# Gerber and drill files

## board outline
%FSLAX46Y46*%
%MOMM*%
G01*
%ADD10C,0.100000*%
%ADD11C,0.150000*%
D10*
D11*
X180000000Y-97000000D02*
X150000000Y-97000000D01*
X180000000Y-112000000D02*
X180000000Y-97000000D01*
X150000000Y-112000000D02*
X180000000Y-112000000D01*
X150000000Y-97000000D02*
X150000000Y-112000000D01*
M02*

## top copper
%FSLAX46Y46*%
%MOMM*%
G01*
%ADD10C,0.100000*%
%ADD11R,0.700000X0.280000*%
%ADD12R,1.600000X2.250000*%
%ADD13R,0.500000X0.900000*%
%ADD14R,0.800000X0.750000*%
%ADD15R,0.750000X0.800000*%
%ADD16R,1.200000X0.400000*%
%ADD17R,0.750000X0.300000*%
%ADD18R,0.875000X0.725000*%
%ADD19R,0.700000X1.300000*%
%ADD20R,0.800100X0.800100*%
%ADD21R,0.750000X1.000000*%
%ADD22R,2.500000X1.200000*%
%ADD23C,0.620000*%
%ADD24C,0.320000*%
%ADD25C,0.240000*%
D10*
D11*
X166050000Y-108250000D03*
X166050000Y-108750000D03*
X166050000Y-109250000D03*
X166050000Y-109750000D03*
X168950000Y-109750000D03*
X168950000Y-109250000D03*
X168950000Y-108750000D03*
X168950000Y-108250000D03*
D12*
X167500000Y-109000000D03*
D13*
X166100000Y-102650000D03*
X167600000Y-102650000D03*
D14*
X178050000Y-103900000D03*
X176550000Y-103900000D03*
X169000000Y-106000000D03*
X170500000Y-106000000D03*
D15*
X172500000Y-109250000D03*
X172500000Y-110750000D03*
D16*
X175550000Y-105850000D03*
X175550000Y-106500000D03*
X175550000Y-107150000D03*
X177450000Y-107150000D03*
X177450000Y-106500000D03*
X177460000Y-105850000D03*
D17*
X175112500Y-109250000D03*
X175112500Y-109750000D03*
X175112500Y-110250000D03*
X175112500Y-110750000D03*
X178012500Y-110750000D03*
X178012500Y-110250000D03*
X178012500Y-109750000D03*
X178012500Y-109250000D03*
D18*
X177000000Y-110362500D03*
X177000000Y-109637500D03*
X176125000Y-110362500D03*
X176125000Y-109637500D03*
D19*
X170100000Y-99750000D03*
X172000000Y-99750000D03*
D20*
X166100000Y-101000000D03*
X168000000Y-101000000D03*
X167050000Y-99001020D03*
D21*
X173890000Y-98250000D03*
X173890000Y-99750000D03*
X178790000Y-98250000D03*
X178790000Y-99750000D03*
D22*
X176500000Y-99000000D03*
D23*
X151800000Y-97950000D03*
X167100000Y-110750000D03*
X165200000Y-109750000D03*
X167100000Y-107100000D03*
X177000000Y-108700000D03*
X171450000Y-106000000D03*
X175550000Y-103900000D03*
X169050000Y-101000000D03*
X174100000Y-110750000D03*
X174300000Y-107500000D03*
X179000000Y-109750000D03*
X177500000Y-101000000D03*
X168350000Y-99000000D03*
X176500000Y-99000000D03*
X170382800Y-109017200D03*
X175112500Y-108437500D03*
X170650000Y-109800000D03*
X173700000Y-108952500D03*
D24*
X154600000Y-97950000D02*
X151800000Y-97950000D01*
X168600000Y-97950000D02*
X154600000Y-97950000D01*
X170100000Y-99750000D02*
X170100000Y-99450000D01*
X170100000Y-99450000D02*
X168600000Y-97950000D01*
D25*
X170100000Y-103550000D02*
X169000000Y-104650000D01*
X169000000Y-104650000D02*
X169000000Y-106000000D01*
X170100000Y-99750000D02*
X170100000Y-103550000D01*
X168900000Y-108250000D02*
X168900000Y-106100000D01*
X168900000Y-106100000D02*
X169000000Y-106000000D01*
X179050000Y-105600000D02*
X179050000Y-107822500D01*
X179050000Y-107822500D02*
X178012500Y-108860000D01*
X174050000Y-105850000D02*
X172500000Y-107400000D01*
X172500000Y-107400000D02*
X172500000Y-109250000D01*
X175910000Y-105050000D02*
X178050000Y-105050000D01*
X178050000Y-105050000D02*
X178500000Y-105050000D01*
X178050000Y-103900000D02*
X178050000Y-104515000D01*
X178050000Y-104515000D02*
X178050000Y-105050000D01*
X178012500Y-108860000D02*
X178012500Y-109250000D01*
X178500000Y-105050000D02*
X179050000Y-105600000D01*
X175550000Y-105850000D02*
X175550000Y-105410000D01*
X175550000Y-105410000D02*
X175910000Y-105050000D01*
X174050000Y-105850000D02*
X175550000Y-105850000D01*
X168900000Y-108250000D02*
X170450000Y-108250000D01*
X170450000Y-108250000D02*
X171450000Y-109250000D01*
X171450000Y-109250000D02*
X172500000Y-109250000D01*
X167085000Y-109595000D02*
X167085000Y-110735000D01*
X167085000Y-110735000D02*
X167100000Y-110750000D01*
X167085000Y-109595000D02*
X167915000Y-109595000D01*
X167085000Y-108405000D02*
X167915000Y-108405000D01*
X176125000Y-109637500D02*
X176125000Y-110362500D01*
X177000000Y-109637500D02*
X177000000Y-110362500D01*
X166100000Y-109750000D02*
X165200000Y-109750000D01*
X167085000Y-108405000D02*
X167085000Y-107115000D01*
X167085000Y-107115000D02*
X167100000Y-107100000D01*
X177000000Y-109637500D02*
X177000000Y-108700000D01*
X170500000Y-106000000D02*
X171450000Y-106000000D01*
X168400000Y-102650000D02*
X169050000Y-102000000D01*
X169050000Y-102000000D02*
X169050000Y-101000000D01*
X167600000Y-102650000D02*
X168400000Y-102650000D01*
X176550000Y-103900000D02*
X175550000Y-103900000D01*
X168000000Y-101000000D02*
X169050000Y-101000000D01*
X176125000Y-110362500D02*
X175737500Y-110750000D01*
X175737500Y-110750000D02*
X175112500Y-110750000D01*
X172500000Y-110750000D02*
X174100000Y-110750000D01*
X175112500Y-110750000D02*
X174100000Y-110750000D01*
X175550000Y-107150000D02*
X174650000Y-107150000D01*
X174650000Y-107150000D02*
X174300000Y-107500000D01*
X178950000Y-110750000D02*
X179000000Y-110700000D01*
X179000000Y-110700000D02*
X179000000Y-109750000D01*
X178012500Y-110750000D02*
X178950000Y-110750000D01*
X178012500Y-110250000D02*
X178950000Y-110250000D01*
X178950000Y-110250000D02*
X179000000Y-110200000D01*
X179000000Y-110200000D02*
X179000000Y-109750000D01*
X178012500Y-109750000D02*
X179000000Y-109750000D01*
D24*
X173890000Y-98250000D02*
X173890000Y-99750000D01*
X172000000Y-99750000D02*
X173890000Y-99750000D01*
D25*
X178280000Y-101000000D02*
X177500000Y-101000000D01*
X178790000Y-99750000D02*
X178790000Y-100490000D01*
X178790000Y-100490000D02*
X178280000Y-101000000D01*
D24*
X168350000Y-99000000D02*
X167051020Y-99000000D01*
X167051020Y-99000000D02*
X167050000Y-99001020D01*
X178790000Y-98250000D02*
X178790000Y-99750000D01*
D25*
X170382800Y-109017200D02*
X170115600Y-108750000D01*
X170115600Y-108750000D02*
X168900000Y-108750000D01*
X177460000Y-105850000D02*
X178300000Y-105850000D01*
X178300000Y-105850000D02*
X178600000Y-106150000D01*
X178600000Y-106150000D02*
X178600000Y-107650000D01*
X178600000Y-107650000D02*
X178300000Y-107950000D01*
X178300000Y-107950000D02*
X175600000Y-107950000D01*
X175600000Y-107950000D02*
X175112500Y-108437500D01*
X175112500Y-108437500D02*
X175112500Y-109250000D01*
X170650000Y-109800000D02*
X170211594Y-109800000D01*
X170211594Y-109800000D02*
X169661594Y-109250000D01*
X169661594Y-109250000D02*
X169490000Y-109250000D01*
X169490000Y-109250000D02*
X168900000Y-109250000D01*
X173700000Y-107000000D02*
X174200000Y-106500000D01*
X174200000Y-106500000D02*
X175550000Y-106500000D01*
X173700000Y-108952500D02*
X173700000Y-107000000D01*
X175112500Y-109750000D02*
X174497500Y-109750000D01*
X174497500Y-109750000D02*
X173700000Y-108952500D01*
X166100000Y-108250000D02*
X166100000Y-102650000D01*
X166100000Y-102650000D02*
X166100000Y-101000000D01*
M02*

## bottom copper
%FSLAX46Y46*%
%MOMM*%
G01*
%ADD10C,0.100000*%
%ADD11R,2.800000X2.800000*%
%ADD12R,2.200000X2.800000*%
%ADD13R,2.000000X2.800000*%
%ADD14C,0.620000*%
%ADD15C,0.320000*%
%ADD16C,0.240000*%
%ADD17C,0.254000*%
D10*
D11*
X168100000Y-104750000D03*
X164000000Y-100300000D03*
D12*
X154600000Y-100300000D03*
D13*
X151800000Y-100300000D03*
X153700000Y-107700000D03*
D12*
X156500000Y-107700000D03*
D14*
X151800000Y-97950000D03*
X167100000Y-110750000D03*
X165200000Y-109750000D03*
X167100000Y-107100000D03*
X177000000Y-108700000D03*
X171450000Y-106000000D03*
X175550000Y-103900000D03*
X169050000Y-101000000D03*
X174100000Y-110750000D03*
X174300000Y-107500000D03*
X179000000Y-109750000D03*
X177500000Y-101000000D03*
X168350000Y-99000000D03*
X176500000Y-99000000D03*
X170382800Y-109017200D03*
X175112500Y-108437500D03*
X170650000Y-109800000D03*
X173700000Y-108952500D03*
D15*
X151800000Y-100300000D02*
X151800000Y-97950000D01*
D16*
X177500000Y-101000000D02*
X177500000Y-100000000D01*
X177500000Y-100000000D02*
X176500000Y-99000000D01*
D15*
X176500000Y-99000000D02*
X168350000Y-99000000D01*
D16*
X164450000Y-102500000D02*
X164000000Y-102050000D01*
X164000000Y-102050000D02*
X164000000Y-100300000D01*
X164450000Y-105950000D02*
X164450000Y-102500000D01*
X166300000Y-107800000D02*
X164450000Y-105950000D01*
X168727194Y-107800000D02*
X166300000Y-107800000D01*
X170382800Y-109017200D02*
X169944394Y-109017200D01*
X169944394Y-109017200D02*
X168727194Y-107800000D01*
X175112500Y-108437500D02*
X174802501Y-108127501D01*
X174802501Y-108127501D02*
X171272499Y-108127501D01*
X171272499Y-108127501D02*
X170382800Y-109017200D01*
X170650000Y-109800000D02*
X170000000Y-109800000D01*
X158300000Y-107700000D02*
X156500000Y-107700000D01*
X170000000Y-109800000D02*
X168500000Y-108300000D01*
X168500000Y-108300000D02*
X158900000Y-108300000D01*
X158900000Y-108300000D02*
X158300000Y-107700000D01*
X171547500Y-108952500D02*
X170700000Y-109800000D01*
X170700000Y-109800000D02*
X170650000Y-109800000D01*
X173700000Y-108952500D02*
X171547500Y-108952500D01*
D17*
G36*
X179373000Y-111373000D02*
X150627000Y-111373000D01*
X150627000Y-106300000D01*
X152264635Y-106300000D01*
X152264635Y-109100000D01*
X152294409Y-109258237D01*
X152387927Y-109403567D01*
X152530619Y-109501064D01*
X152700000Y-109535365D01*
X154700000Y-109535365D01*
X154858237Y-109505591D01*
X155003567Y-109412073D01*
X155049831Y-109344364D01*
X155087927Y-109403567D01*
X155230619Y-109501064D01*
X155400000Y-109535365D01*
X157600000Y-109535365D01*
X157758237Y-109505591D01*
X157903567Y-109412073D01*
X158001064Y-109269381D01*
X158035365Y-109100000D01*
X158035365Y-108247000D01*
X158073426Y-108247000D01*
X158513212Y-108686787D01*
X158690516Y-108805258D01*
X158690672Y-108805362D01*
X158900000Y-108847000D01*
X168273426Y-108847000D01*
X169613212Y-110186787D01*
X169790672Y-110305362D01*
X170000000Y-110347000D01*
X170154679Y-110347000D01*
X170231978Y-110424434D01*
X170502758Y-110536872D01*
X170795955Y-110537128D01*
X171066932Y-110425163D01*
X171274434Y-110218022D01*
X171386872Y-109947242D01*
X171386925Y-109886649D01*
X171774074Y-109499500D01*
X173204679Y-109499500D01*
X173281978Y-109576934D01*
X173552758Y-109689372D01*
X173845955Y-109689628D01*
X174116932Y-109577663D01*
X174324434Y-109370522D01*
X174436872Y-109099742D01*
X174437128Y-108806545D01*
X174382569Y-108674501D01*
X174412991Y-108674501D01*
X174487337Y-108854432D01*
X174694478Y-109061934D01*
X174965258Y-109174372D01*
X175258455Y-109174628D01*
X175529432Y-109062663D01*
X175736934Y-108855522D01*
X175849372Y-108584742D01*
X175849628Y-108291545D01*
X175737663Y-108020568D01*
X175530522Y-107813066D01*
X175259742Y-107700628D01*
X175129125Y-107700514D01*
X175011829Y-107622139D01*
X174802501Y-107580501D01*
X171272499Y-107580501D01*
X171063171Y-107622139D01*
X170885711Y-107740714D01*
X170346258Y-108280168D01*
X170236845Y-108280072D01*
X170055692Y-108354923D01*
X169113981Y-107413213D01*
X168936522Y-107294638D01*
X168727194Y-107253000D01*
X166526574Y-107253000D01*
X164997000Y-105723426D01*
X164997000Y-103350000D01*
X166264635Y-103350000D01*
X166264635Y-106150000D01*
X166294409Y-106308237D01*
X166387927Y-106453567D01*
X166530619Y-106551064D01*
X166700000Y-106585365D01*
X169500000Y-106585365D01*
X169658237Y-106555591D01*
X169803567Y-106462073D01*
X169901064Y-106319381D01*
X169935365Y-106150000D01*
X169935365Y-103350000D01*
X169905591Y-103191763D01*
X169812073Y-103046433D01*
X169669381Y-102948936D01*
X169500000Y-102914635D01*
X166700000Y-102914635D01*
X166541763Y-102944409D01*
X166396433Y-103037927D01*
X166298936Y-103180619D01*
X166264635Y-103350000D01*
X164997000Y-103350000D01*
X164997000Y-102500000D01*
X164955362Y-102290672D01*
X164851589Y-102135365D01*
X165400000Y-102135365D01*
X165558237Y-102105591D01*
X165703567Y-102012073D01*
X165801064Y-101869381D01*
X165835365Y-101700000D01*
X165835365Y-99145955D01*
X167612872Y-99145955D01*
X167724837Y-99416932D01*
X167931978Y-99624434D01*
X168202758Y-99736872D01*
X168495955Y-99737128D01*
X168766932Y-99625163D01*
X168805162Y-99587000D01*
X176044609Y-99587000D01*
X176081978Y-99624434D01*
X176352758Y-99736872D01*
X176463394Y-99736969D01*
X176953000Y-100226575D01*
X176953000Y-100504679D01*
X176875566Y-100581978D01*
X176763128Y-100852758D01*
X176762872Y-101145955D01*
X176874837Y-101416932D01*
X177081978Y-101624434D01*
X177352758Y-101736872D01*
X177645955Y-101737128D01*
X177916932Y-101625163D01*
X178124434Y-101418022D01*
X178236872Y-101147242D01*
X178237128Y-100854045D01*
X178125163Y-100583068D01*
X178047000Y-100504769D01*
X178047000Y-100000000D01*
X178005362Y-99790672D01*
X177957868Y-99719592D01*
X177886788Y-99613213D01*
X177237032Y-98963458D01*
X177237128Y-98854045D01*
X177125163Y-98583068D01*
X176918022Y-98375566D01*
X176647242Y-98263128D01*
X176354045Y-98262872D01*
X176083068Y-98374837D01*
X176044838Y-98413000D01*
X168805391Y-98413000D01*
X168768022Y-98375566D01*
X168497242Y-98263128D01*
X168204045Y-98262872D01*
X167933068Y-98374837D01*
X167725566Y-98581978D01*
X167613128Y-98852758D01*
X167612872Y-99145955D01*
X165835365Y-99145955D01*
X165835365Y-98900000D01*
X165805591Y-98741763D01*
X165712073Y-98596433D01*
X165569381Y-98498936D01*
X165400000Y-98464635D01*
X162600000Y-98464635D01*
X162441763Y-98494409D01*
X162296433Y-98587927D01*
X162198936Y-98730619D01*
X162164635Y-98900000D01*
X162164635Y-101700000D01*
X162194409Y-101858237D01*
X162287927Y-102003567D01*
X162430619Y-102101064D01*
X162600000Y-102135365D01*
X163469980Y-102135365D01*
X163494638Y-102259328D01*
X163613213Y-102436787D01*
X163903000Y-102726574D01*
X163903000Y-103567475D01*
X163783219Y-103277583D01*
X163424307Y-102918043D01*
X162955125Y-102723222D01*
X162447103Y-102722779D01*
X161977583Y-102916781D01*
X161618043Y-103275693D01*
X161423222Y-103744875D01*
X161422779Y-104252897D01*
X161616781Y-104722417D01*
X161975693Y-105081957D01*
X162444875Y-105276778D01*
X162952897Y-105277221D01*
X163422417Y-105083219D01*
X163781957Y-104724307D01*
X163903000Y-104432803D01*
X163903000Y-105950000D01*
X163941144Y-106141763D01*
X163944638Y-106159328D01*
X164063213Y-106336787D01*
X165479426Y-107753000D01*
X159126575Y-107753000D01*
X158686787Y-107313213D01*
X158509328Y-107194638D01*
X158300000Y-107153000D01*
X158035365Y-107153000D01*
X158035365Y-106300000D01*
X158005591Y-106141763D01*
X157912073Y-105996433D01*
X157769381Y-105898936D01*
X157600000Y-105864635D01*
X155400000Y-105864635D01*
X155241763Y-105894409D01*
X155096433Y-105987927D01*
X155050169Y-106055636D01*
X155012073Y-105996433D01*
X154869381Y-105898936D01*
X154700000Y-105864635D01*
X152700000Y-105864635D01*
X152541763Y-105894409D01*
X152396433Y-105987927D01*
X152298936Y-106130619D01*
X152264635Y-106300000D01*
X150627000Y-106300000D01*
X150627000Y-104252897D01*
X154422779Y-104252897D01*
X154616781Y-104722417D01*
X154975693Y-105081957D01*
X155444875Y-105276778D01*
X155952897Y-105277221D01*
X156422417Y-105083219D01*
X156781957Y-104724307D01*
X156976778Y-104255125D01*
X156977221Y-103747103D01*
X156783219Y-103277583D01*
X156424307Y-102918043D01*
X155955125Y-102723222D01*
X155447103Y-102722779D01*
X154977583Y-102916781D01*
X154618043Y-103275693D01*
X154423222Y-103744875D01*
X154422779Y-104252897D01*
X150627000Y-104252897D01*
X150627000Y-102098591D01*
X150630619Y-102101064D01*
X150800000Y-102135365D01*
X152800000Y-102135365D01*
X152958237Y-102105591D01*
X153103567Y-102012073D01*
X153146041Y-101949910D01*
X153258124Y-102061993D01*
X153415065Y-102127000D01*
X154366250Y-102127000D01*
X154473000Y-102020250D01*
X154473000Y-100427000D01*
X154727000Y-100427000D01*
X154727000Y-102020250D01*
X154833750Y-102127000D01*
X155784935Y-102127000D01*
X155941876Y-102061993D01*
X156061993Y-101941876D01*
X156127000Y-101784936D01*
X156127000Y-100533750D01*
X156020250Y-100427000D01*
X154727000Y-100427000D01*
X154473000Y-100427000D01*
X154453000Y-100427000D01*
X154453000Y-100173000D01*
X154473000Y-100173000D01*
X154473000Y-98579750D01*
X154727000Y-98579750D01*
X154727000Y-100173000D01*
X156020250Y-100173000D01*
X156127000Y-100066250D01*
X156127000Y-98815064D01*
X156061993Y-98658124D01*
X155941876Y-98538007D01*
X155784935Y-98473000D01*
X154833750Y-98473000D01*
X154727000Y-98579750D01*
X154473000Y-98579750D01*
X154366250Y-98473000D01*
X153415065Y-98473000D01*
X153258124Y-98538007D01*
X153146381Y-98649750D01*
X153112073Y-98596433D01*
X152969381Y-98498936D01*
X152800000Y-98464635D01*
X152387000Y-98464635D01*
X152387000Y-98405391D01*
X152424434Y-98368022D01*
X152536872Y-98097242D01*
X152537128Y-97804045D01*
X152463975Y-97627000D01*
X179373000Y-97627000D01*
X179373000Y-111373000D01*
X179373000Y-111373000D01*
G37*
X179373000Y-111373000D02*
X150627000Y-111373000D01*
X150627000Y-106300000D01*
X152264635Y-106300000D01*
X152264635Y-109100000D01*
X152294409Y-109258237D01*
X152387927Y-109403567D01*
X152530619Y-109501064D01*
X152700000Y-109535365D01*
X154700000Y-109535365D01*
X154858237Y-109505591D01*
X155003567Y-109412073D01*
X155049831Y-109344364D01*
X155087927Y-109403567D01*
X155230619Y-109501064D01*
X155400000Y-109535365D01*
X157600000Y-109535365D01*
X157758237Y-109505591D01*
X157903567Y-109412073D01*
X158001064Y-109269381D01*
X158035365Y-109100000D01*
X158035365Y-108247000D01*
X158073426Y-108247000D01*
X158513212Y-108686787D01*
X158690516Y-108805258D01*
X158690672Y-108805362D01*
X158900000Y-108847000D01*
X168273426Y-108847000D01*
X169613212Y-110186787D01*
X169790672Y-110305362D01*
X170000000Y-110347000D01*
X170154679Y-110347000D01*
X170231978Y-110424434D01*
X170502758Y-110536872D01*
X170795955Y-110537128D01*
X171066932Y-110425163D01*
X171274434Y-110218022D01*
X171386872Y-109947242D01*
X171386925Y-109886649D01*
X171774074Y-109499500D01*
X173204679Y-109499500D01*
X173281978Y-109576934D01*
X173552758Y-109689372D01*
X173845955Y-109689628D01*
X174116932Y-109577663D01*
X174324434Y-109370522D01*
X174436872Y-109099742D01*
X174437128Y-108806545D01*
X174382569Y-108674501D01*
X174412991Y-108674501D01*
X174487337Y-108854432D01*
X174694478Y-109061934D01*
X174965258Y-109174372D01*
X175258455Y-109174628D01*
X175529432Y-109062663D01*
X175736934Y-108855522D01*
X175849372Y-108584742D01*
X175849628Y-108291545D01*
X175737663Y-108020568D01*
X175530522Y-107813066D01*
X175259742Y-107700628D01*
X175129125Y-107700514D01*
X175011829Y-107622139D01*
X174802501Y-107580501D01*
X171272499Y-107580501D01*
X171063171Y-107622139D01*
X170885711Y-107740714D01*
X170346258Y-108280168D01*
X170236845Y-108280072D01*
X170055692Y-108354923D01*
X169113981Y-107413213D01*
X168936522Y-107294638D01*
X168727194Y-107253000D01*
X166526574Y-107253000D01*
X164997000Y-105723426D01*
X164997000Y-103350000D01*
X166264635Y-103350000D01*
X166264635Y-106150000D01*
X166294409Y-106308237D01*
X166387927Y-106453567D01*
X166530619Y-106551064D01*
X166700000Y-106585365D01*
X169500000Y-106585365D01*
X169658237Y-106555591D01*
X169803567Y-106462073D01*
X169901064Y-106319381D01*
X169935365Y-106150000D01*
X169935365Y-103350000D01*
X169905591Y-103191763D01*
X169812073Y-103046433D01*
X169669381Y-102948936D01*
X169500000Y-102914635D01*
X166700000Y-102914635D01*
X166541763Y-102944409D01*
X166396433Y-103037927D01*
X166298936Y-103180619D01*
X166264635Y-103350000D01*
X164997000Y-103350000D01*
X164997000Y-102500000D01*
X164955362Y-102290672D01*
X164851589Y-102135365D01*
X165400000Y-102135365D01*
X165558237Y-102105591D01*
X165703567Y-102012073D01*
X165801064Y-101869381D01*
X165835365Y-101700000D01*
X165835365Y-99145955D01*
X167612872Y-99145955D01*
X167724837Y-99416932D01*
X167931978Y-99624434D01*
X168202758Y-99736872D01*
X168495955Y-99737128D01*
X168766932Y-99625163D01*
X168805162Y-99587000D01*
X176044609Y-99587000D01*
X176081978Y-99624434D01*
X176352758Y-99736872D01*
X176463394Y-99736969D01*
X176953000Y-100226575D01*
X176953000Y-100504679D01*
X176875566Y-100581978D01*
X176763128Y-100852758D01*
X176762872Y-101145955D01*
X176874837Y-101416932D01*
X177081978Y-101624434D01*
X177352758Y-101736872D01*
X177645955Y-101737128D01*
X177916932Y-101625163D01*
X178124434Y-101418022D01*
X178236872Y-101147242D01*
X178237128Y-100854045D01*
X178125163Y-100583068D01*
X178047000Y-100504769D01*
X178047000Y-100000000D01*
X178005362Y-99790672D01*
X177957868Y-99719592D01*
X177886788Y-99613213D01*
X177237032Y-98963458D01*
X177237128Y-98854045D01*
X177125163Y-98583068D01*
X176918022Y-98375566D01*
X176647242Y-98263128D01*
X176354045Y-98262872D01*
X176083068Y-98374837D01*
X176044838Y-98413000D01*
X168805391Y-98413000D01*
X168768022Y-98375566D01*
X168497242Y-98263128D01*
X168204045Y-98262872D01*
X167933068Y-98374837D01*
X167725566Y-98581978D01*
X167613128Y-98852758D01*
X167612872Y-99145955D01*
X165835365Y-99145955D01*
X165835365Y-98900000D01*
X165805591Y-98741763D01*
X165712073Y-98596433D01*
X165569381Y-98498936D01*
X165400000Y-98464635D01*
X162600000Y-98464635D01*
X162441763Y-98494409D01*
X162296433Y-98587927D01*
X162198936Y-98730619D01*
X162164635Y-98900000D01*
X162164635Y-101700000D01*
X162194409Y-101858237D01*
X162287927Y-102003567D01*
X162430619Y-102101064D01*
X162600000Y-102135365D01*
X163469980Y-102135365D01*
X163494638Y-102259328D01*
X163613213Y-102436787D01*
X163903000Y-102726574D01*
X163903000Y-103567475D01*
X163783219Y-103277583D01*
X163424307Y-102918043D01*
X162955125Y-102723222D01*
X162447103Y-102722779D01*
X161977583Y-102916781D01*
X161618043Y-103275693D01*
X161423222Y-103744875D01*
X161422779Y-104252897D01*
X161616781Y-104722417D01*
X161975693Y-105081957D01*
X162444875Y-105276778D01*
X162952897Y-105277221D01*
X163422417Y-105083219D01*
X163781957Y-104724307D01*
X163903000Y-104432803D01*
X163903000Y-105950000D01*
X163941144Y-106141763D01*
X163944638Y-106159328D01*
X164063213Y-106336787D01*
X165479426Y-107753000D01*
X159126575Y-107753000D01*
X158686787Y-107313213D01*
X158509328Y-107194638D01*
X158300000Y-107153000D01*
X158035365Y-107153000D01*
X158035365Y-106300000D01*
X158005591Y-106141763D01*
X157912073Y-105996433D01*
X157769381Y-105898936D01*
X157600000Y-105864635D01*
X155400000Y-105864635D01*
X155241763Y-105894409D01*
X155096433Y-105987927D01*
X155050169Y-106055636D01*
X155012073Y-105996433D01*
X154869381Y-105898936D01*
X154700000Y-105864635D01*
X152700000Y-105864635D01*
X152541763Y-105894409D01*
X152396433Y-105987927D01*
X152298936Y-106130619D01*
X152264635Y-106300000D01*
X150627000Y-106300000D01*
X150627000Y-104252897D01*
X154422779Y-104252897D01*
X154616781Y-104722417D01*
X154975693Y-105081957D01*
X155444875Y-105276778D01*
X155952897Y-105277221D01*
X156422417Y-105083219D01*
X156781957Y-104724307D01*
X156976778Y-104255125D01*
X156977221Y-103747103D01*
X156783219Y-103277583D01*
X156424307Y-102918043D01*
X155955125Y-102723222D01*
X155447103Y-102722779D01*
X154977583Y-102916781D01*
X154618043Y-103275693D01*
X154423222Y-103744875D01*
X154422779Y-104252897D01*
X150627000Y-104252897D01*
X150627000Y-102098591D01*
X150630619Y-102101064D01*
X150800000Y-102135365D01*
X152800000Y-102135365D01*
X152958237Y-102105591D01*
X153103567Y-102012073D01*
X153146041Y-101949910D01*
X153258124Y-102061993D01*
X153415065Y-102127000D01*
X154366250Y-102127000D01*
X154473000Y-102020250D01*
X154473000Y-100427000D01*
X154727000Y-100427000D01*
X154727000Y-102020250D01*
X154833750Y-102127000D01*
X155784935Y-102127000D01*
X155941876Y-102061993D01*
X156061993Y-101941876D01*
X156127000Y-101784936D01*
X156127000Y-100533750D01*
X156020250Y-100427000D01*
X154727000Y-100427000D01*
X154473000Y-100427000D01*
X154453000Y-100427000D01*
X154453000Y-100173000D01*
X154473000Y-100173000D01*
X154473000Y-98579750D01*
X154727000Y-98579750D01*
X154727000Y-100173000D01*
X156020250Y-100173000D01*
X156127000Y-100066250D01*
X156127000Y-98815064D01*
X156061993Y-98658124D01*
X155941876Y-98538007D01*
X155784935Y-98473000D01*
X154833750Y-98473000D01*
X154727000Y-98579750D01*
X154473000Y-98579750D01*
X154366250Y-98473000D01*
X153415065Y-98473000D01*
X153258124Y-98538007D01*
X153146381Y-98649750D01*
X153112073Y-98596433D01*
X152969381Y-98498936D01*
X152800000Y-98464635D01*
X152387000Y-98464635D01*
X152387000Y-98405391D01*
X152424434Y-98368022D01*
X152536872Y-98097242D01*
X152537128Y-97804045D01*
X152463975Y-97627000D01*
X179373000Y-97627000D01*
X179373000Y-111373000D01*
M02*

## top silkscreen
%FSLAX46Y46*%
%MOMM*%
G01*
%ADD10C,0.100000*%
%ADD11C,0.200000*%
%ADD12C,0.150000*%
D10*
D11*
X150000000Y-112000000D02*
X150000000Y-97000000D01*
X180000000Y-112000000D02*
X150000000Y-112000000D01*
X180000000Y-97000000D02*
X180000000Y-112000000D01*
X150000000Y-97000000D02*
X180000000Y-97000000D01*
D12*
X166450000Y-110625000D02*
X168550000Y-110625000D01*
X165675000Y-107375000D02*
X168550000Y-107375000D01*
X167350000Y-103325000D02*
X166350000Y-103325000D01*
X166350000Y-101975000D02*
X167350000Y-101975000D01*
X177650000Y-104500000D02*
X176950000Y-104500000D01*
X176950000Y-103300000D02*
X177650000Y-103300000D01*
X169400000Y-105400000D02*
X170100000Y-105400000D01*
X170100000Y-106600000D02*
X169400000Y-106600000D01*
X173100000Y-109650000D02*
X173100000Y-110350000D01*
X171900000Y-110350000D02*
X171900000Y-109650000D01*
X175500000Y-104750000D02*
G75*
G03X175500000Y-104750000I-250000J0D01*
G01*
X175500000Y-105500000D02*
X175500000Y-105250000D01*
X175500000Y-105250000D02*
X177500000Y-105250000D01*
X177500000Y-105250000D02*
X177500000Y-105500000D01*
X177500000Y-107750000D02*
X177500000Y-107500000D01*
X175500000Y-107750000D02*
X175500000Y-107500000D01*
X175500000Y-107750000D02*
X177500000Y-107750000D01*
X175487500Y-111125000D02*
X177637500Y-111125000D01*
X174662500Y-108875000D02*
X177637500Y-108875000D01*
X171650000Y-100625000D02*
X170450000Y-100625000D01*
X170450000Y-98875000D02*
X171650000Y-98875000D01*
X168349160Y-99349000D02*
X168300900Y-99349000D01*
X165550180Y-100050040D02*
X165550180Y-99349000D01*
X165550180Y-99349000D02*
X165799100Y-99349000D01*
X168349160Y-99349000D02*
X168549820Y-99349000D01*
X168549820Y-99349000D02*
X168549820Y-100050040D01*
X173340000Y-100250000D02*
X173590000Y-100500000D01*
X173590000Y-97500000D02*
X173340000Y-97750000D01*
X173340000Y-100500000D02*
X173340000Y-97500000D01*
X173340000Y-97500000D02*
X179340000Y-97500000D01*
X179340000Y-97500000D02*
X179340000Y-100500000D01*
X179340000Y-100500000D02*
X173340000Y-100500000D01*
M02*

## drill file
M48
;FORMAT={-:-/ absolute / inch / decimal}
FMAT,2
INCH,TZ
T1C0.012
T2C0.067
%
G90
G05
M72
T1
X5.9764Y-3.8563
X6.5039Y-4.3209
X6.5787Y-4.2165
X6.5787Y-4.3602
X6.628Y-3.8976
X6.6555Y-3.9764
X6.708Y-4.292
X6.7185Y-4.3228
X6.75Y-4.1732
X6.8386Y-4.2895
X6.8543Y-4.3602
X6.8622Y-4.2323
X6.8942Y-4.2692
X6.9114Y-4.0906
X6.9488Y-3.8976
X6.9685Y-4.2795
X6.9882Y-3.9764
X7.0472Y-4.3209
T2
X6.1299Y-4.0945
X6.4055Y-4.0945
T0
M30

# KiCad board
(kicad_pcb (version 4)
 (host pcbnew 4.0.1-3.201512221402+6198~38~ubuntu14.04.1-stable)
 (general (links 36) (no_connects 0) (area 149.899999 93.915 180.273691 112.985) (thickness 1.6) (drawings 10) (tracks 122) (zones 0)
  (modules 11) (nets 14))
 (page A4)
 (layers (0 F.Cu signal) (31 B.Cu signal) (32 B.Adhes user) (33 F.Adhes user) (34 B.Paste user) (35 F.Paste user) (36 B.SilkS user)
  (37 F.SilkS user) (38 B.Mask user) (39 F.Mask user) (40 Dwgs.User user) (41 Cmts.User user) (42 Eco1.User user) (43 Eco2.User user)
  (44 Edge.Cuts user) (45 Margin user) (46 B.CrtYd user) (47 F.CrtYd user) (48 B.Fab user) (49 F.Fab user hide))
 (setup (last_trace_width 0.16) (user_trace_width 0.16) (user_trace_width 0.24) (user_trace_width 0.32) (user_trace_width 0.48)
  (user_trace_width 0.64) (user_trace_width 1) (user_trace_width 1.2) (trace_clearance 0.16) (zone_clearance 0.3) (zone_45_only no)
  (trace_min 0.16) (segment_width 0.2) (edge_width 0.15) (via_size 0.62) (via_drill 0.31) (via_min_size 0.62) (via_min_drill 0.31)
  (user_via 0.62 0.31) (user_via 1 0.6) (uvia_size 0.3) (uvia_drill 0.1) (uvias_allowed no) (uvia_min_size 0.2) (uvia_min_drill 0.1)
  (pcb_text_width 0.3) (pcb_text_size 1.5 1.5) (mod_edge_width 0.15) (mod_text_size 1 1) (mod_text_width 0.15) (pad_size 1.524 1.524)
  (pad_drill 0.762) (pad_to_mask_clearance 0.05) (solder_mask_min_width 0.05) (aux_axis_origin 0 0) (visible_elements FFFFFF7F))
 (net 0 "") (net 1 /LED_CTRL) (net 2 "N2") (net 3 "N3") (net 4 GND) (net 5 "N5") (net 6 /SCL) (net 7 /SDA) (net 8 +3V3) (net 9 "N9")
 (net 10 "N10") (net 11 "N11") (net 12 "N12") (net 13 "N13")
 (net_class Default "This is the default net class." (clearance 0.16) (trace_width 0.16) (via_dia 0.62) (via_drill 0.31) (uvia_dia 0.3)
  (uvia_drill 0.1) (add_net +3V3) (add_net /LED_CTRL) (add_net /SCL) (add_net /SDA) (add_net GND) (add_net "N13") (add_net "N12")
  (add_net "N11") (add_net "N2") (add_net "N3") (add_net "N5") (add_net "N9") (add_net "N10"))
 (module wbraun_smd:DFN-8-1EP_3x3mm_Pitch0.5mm (layer F.Cu) (at 167.5 109)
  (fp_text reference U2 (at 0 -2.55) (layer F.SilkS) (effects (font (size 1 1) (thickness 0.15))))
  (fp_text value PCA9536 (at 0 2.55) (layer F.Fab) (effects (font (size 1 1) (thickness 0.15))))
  (fp_line (start -1.05 1.625) (end 1.05 1.625) (layer F.SilkS) (width 0.15))
  (fp_line (start -1.825 -1.625) (end 1.05 -1.625) (layer F.SilkS) (width 0.15))
  (pad 1 smd rect (at -1.45 -0.75) (size 0.7 0.28) (layers F.Cu F.Paste F.Mask) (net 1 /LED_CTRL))
  (pad 2 smd rect (at -1.45 -0.25) (size 0.7 0.28) (layers F.Cu F.Paste F.Mask) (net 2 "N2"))
  (pad 3 smd rect (at -1.45 0.25) (size 0.7 0.28) (layers F.Cu F.Paste F.Mask) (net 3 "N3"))
  (pad 4 smd rect (at -1.45 0.75) (size 0.7 0.28) (layers F.Cu F.Paste F.Mask) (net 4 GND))
  (pad 5 smd rect (at 1.45 0.75) (size 0.7 0.28) (layers F.Cu F.Paste F.Mask) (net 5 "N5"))
  (pad 6 smd rect (at 1.45 0.25) (size 0.7 0.28) (layers F.Cu F.Paste F.Mask) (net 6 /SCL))
  (pad 7 smd rect (at 1.45 -0.25) (size 0.7 0.28) (layers F.Cu F.Paste F.Mask) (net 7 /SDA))
  (pad 8 smd rect (at 1.45 -0.75) (size 0.7 0.28) (layers F.Cu F.Paste F.Mask) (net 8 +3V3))
  (pad 9 smd rect (at 0 0) (size 1.6 2.25) (layers F.Cu F.Paste F.Mask) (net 4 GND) (solder_paste_margin_ratio -0.2)))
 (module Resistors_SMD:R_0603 (layer F.Cu) (at 166.85 102.65)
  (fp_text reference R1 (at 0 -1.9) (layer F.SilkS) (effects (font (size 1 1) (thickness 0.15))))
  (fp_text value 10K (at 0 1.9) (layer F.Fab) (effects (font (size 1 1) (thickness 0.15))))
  (fp_line (start 0.5 0.675) (end -0.5 0.675) (layer F.SilkS) (width 0.15))
  (fp_line (start -0.5 -0.675) (end 0.5 -0.675) (layer F.SilkS) (width 0.15))
  (pad 1 smd rect (at -0.75 0) (size 0.5 0.9) (layers F.Cu F.Paste F.Mask) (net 1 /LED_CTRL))
  (pad 2 smd rect (at 0.75 0) (size 0.5 0.9) (layers F.Cu F.Paste F.Mask) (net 4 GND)))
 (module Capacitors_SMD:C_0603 (layer F.Cu) (at 177.3 103.9 180)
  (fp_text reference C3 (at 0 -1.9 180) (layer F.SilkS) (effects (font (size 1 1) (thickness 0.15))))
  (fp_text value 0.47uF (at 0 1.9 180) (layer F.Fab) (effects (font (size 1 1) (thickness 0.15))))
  (fp_line (start -0.35 -0.6) (end 0.35 -0.6) (layer F.SilkS) (width 0.15))
  (fp_line (start 0.35 0.6) (end -0.35 0.6) (layer F.SilkS) (width 0.15))
  (pad 1 smd rect (at -0.75 0 180) (size 0.8 0.75) (layers F.Cu F.Paste F.Mask) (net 8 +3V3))
  (pad 2 smd rect (at 0.75 0 180) (size 0.8 0.75) (layers F.Cu F.Paste F.Mask) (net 4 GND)))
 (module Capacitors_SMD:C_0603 (layer F.Cu) (at 169.75 106)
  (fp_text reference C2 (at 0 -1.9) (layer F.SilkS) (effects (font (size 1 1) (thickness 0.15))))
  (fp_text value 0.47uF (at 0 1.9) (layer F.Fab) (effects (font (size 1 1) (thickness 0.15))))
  (fp_line (start -0.35 -0.6) (end 0.35 -0.6) (layer F.SilkS) (width 0.15))
  (fp_line (start 0.35 0.6) (end -0.35 0.6) (layer F.SilkS) (width 0.15))
  (pad 1 smd rect (at -0.75 0) (size 0.8 0.75) (layers F.Cu F.Paste F.Mask) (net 8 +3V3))
  (pad 2 smd rect (at 0.75 0) (size 0.8 0.75) (layers F.Cu F.Paste F.Mask) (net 4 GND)))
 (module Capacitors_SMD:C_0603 (layer F.Cu) (at 172.5 110 270)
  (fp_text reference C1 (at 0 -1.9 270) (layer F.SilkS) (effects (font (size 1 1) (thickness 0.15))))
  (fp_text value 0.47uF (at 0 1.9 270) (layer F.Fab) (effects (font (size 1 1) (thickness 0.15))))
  (fp_line (start -0.35 -0.6) (end 0.35 -0.6) (layer F.SilkS) (width 0.15))
  (fp_line (start 0.35 0.6) (end -0.35 0.6) (layer F.SilkS) (width 0.15))
  (pad 1 smd rect (at -0.75 0 270) (size 0.8 0.75) (layers F.Cu F.Paste F.Mask) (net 8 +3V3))
  (pad 2 smd rect (at 0.75 0 270) (size 0.8 0.75) (layers F.Cu F.Paste F.Mask) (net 4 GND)))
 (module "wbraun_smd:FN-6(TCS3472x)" (layer F.Cu) (at 176.5 106.5)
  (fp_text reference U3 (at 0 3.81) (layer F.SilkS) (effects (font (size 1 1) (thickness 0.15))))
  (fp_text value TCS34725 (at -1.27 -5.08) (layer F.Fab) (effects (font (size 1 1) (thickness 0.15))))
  (fp_circle (center -1.25 -1.75) (end -1.25 -1.5) (layer F.SilkS) (width 0.15))
  (fp_line (start -1 -1) (end -1 -1.25) (layer F.SilkS) (width 0.15))
  (fp_line (start -1 -1.25) (end 1 -1.25) (layer F.SilkS) (width 0.15))
  (fp_line (start 1 -1.25) (end 1 -1) (layer F.SilkS) (width 0.15))
  (fp_line (start 1 1.25) (end 1 1) (layer F.SilkS) (width 0.15))
  (fp_line (start -1 1.25) (end -1 1) (layer F.SilkS) (width 0.15))
  (fp_line (start -1 1.25) (end 1 1.25) (layer F.SilkS) (width 0.15))
  (pad 1 smd rect (at -0.95 -0.65) (size 1.2 0.4) (layers F.Cu F.Paste F.Mask) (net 8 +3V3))
  (pad 2 smd rect (at -0.95 0) (size 1.2 0.4) (layers F.Cu F.Paste F.Mask) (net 6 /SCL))
  (pad 3 smd rect (at -0.95 0.65) (size 1.2 0.4) (layers F.Cu F.Paste F.Mask) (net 4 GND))
  (pad 4 smd rect (at 0.95 0.65) (size 1.2 0.4) (layers F.Cu F.Paste F.Mask) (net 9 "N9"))
  (pad 5 smd rect (at 0.95 0) (size 1.2 0.4) (layers F.Cu F.Paste F.Mask) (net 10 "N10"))
  (pad 6 smd rect (at 0.96 -0.65) (size 1.2 0.4) (layers F.Cu F.Paste F.Mask) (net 7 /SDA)))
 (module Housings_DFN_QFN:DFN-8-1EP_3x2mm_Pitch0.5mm (layer F.Cu) (at 176.5625 110)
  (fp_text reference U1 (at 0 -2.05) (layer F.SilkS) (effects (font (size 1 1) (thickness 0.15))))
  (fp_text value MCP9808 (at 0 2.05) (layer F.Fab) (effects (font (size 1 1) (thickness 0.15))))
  (fp_line (start -1.075 1.125) (end 1.075 1.125) (layer F.SilkS) (width 0.15))
  (fp_line (start -1.9 -1.125) (end 1.075 -1.125) (layer F.SilkS) (width 0.15))
  (pad 1 smd rect (at -1.45 -0.75) (size 0.75 0.3) (layers F.Cu F.Paste F.Mask) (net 7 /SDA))
  (pad 2 smd rect (at -1.45 -0.25) (size 0.75 0.3) (layers F.Cu F.Paste F.Mask) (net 6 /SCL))
  (pad 3 smd rect (at -1.45 0.25) (size 0.75 0.3) (layers F.Cu F.Paste F.Mask) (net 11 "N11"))
  (pad 4 smd rect (at -1.45 0.75) (size 0.75 0.3) (layers F.Cu F.Paste F.Mask) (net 4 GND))
  (pad 5 smd rect (at 1.45 0.75) (size 0.75 0.3) (layers F.Cu F.Paste F.Mask) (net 4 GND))
  (pad 6 smd rect (at 1.45 0.25) (size 0.75 0.3) (layers F.Cu F.Paste F.Mask) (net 4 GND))
  (pad 7 smd rect (at 1.45 -0.25) (size 0.75 0.3) (layers F.Cu F.Paste F.Mask) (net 4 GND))
  (pad 8 smd rect (at 1.45 -0.75) (size 0.75 0.3) (layers F.Cu F.Paste F.Mask) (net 8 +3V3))
  (pad 9 smd rect (at 0.4375 0.3625) (size 0.875 0.725) (layers F.Cu F.Paste F.Mask) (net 4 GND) (solder_paste_margin_ratio -0.2))
  (pad 9 smd rect (at 0.4375 -0.3625) (size 0.875 0.725) (layers F.Cu F.Paste F.Mask) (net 4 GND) (solder_paste_margin_ratio -0.2))
  (pad 9 smd rect (at -0.4375 0.3625) (size 0.875 0.725) (layers F.Cu F.Paste F.Mask) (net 4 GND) (solder_paste_margin_ratio -0.2))
  (pad 9 smd rect (at -0.4375 -0.3625) (size 0.875 0.725) (layers F.Cu F.Paste F.Mask) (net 4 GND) (solder_paste_margin_ratio -0.2)))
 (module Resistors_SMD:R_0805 (layer F.Cu) (at 171.05 99.75)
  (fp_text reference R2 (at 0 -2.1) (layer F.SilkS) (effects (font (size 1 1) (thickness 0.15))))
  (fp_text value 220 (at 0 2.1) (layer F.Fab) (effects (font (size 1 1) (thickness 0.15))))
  (fp_line (start 0.6 0.875) (end -0.6 0.875) (layer F.SilkS) (width 0.15))
  (fp_line (start -0.6 -0.875) (end 0.6 -0.875) (layer F.SilkS) (width 0.15))
  (pad 1 smd rect (at -0.95 0) (size 0.7 1.3) (layers F.Cu F.Paste F.Mask) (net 8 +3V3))
  (pad 2 smd rect (at 0.95 0) (size 0.7 1.3) (layers F.Cu F.Paste F.Mask) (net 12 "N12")))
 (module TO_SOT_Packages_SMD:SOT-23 (layer F.Cu) (at 167.05 99.99924)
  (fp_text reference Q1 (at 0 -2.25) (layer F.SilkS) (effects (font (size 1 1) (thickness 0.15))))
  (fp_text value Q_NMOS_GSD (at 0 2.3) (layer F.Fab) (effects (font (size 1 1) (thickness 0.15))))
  (fp_line (start 1.29916 -0.65024) (end 1.2509 -0.65024) (layer F.SilkS) (width 0.15))
  (fp_line (start -1.49982 0.0508) (end -1.49982 -0.65024) (layer F.SilkS) (width 0.15))
  (fp_line (start -1.49982 -0.65024) (end -1.2509 -0.65024) (layer F.SilkS) (width 0.15))
  (fp_line (start 1.29916 -0.65024) (end 1.49982 -0.65024) (layer F.SilkS) (width 0.15))
  (fp_line (start 1.49982 -0.65024) (end 1.49982 0.0508) (layer F.SilkS) (width 0.15))
  (pad 1 smd rect (at -0.95 1.00076) (size 0.8001 0.8001) (layers F.Cu F.Paste F.Mask) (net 1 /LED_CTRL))
  (pad 2 smd rect (at 0.95 1.00076) (size 0.8001 0.8001) (layers F.Cu F.Paste F.Mask) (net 4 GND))
  (pad 3 smd rect (at 0 -0.99822) (size 0.8001 0.8001) (layers F.Cu F.Paste F.Mask) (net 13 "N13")))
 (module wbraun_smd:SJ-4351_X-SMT (layer B.Cu) (at 162.1 104)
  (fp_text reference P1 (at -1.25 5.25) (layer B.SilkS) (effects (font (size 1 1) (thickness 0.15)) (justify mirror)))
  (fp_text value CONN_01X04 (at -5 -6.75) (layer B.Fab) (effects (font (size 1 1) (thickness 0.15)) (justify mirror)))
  (pad 5 smd rect (at 6 0.75) (size 2.8 2.8) (layers B.Cu B.Paste B.Mask))
  (pad 2 smd rect (at 1.9 -3.7) (size 2.8 2.8) (layers B.Cu B.Paste B.Mask) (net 7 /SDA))
  (pad 4 smd rect (at -7.5 -3.7) (size 2.2 2.8) (layers B.Cu B.Paste B.Mask) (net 4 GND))
  (pad 1 smd rect (at -10.3 -3.7) (size 2 2.8) (layers B.Cu B.Paste B.Mask) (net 8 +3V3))
  (pad 6 smd rect (at -8.4 3.7) (size 2 2.8) (layers B.Cu B.Paste B.Mask))
  (pad 3 smd rect (at -5.6 3.7) (size 2.2 2.8) (layers B.Cu B.Paste B.Mask) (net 6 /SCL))
  (pad "" np_thru_hole circle (at -6.4 0) (size 1.7 1.7) (drill 1.7) (layers *.Cu *.Mask B.SilkS))
  (pad "" np_thru_hole circle (at 0.6 0) (size 1.7 1.7) (drill 1.7) (layers *.Cu *.Mask B.SilkS)))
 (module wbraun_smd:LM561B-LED (layer F.Cu) (at 176.34 99)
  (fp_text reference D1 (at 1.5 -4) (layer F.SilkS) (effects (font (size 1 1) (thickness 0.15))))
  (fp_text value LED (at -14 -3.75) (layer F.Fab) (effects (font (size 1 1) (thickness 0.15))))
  (fp_line (start -3 1.25) (end -2.75 1.5) (layer F.SilkS) (width 0.15))
  (fp_line (start -2.75 -1.5) (end -3 -1.25) (layer F.SilkS) (width 0.15))
  (fp_line (start -3 1.5) (end -3 -1.5) (layer F.SilkS) (width 0.15))
  (fp_line (start -3 -1.5) (end 3 -1.5) (layer F.SilkS) (width 0.15))
  (fp_line (start 3 -1.5) (end 3 1.5) (layer F.SilkS) (width 0.15))
  (fp_line (start 3 1.5) (end -3 1.5) (layer F.SilkS) (width 0.15))
  (pad 2 smd rect (at -2.45 -0.75) (size 0.75 1) (layers F.Cu F.Paste F.Mask) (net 12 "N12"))
  (pad 2 smd rect (at -2.45 0.75) (size 0.75 1) (layers F.Cu F.Paste F.Mask) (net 12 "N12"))
  (pad 1 smd rect (at 2.45 -0.75) (size 0.75 1) (layers F.Cu F.Paste F.Mask) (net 13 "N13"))
  (pad 1 smd rect (at 2.45 0.75) (size 0.75 1) (layers F.Cu F.Paste F.Mask) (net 13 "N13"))
  (pad 1 smd rect (at 0.16 0) (size 2.5 1.2) (layers F.Cu F.Paste F.Mask) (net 13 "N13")))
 (gr_line (start 180 97) (end 150 97) (layer Edge.Cuts) (width 0.15))
 (gr_line (start 180 112) (end 180 97) (layer Edge.Cuts) (width 0.15))
 (gr_line (start 150 112) (end 180 112) (layer Edge.Cuts) (width 0.15))
 (gr_line (start 150 97) (end 150 112) (layer Edge.Cuts) (width 0.15))
 (gr_line (start 150 112) (end 150 97) (angle 90) (layer F.SilkS) (width 0.2))
 (gr_line (start 180 112) (end 150 112) (angle 90) (layer F.SilkS) (width 0.2))
 (gr_line (start 180 97) (end 180 112) (angle 90) (layer F.SilkS) (width 0.2))
 (gr_line (start 150 97) (end 180 97) (angle 90) (layer F.SilkS) (width 0.2))
 (segment (start 151.8 100.3) (end 151.8 97.95) (width 0.32) (layer B.Cu) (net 8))
 (via (at 151.8 97.95) (size 0.62) (drill 0.31) (layers F.Cu B.Cu) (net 8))
 (segment (start 154.6 97.95) (end 151.8 97.95) (width 0.32) (layer F.Cu) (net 8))
 (segment (start 168.6 97.95) (end 154.6 97.95) (width 0.32) (layer F.Cu) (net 8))
 (segment (start 170.1 99.75) (end 170.1 99.45) (width 0.32) (layer F.Cu) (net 8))
 (segment (start 170.1 99.45) (end 168.6 97.95) (width 0.32) (layer F.Cu) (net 8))
 (segment (start 170.1 103.55) (end 169 104.65) (width 0.24) (layer F.Cu) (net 8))
 (segment (start 169 104.65) (end 169 106) (width 0.24) (layer F.Cu) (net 8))
 (segment (start 170.1 99.75) (end 170.1 103.55) (width 0.24) (layer F.Cu) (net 8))
 (segment (start 168.9 108.25) (end 168.9 106.1) (width 0.24) (layer F.Cu) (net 8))
 (segment (start 168.9 106.1) (end 169 106) (width 0.24) (layer F.Cu) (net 8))
 (segment (start 179.05 105.6) (end 179.05 107.8225) (width 0.24) (layer F.Cu) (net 8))
 (segment (start 179.05 107.8225) (end 178.0125 108.86) (width 0.24) (layer F.Cu) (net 8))
 (segment (start 174.05 105.85) (end 172.5 107.4) (width 0.24) (layer F.Cu) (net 8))
 (segment (start 172.5 107.4) (end 172.5 109.25) (width 0.24) (layer F.Cu) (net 8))
 (segment (start 175.91 105.05) (end 178.05 105.05) (width 0.24) (layer F.Cu) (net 8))
 (segment (start 178.05 105.05) (end 178.5 105.05) (width 0.24) (layer F.Cu) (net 8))
 (segment (start 178.05 103.9) (end 178.05 104.515) (width 0.24) (layer F.Cu) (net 8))
 (segment (start 178.05 104.515) (end 178.05 105.05) (width 0.24) (layer F.Cu) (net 8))
 (segment (start 178.0125 108.86) (end 178.0125 109.25) (width 0.24) (layer F.Cu) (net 8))
 (segment (start 178.5 105.05) (end 179.05 105.6) (width 0.24) (layer F.Cu) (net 8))
 (segment (start 175.55 105.85) (end 175.55 105.41) (width 0.24) (layer F.Cu) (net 8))
 (segment (start 175.55 105.41) (end 175.91 105.05) (width 0.24) (layer F.Cu) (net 8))
 (segment (start 174.05 105.85) (end 175.55 105.85) (width 0.24) (layer F.Cu) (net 8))
 (segment (start 168.9 108.25) (end 170.45 108.25) (width 0.24) (layer F.Cu) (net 8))
 (segment (start 170.45 108.25) (end 171.45 109.25) (width 0.24) (layer F.Cu) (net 8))
 (segment (start 171.45 109.25) (end 172.5 109.25) (width 0.24) (layer F.Cu) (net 8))
 (segment (start 167.085 109.595) (end 167.085 110.735) (width 0.24) (layer F.Cu) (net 4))
 (segment (start 167.085 110.735) (end 167.1 110.75) (width 0.24) (layer F.Cu) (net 4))
 (via (at 167.1 110.75) (size 0.62) (drill 0.31) (layers F.Cu B.Cu) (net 4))
 (segment (start 167.085 109.595) (end 167.915 109.595) (width 0.24) (layer F.Cu) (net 4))
 (segment (start 167.085 108.405) (end 167.915 108.405) (width 0.24) (layer F.Cu) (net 4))
 (segment (start 176.125 109.6375) (end 176.125 110.3625) (width 0.24) (layer F.Cu) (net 4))
 (segment (start 177 109.6375) (end 177 110.3625) (width 0.24) (layer F.Cu) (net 4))
 (segment (start 166.1 109.75) (end 165.2 109.75) (width 0.24) (layer F.Cu) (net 4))
 (via (at 165.2 109.75) (size 0.62) (drill 0.31) (layers F.Cu B.Cu) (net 4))
 (segment (start 167.085 108.405) (end 167.085 107.115) (width 0.24) (layer F.Cu) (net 4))
 (segment (start 167.085 107.115) (end 167.1 107.1) (width 0.24) (layer F.Cu) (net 4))
 (via (at 167.1 107.1) (size 0.62) (drill 0.31) (layers F.Cu B.Cu) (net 4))
 (segment (start 177 109.6375) (end 177 108.7) (width 0.24) (layer F.Cu) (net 4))
 (via (at 177 108.7) (size 0.62) (drill 0.31) (layers F.Cu B.Cu) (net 4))
 (segment (start 170.5 106) (end 171.45 106) (width 0.24) (layer F.Cu) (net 4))
 (via (at 171.45 106) (size 0.62) (drill 0.31) (layers F.Cu B.Cu) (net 4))
 (segment (start 168.4 102.65) (end 169.05 102) (width 0.24) (layer F.Cu) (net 4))
 (segment (start 169.05 102) (end 169.05 101) (width 0.24) (layer F.Cu) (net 4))
 (segment (start 167.6 102.65) (end 168.4 102.65) (width 0.24) (layer F.Cu) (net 4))
 (segment (start 176.55 103.9) (end 175.55 103.9) (width 0.24) (layer F.Cu) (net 4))
 (via (at 175.55 103.9) (size 0.62) (drill 0.31) (layers F.Cu B.Cu) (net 4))
 (segment (start 168 101) (end 169.05 101) (width 0.24) (layer F.Cu) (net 4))
 (via (at 169.05 101) (size 0.62) (drill 0.31) (layers F.Cu B.Cu) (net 4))
 (segment (start 176.125 110.3625) (end 175.7375 110.75) (width 0.24) (layer F.Cu) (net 4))
 (segment (start 175.7375 110.75) (end 175.1125 110.75) (width 0.24) (layer F.Cu) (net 4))
 (segment (start 172.5 110.75) (end 174.1 110.75) (width 0.24) (layer F.Cu) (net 4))
 (segment (start 175.1125 110.75) (end 174.1 110.75) (width 0.24) (layer F.Cu) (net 4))
 (via (at 174.1 110.75) (size 0.62) (drill 0.31) (layers F.Cu B.Cu) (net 4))
 (segment (start 175.55 107.15) (end 174.65 107.15) (width 0.24) (layer F.Cu) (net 4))
 (segment (start 174.65 107.15) (end 174.3 107.5) (width 0.24) (layer F.Cu) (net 4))
 (via (at 174.3 107.5) (size 0.62) (drill 0.31) (layers F.Cu B.Cu) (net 4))
 (segment (start 178.95 110.75) (end 179 110.7) (width 0.24) (layer F.Cu) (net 4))
 (segment (start 179 110.7) (end 179 109.75) (width 0.24) (layer F.Cu) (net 4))
 (segment (start 178.0125 110.75) (end 178.95 110.75) (width 0.24) (layer F.Cu) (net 4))
 (segment (start 178.0125 110.25) (end 178.95 110.25) (width 0.24) (layer F.Cu) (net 4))
 (segment (start 178.95 110.25) (end 179 110.2) (width 0.24) (layer F.Cu) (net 4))
 (segment (start 179 110.2) (end 179 109.75) (width 0.24) (layer F.Cu) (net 4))
 (segment (start 178.0125 109.75) (end 179 109.75) (width 0.24) (layer F.Cu) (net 4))
 (via (at 179 109.75) (size 0.62) (drill 0.31) (layers F.Cu B.Cu) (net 4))
 (segment (start 173.89 98.25) (end 173.89 99.75) (width 0.32) (layer F.Cu) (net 12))
 (segment (start 172 99.75) (end 173.89 99.75) (width 0.32) (layer F.Cu) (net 12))
 (segment (start 177.5 101) (end 177.5 100) (width 0.24) (layer B.Cu) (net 13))
 (segment (start 177.5 100) (end 176.5 99) (width 0.24) (layer B.Cu) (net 13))
 (segment (start 178.28 101) (end 177.5 101) (width 0.24) (layer F.Cu) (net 13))
 (via (at 177.5 101) (size 0.62) (drill 0.31) (layers F.Cu B.Cu) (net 13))
 (segment (start 178.79 99.75) (end 178.79 100.49) (width 0.24) (layer F.Cu) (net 13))
 (segment (start 178.79 100.49) (end 178.28 101) (width 0.24) (layer F.Cu) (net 13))
 (segment (start 168.35 99) (end 167.05102 99) (width 0.32) (layer F.Cu) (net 13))
 (segment (start 167.05102 99) (end 167.05 99.00102) (width 0.32) (layer F.Cu) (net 13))
 (segment (start 176.5 99) (end 168.35 99) (width 0.32) (layer B.Cu) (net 13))
 (via (at 168.35 99) (size 0.62) (drill 0.31) (layers F.Cu B.Cu) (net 13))
 (segment (start 178.79 98.25) (end 178.79 99.75) (width 0.32) (layer F.Cu) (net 13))
 (via (at 176.5 99) (size 0.62) (drill 0.31) (layers F.Cu B.Cu) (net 13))
 (segment (start 164.45 102.5) (end 164 102.05) (width 0.24) (layer B.Cu) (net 7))
 (segment (start 164 102.05) (end 164 100.3) (width 0.24) (layer B.Cu) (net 7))
 (segment (start 164.45 105.95) (end 164.45 102.5) (width 0.24) (layer B.Cu) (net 7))
 (segment (start 166.3 107.8) (end 164.45 105.95) (width 0.24) (layer B.Cu) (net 7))
 (segment (start 168.727194 107.8) (end 166.3 107.8) (width 0.24) (layer B.Cu) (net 7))
 (segment (start 170.3828 109.0172) (end 169.944394 109.0172) (width 0.24) (layer B.Cu) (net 7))
 (segment (start 169.944394 109.0172) (end 168.727194 107.8) (width 0.24) (layer B.Cu) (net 7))
 (segment (start 170.3828 109.0172) (end 170.1156 108.75) (width 0.24) (layer F.Cu) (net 7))
 (segment (start 170.1156 108.75) (end 168.9 108.75) (width 0.24) (layer F.Cu) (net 7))
 (segment (start 175.1125 108.4375) (end 174.802501 108.127501) (width 0.24) (layer B.Cu) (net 7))
 (segment (start 174.802501 108.127501) (end 171.272499 108.127501) (width 0.24) (layer B.Cu) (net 7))
 (segment (start 171.272499 108.127501) (end 170.3828 109.0172) (width 0.24) (layer B.Cu) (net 7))
 (via (at 170.3828 109.0172) (size 0.62) (drill 0.31) (layers F.Cu B.Cu) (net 7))
 (via (at 175.1125 108.4375) (size 0.62) (drill 0.31) (layers F.Cu B.Cu) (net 7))
 (segment (start 177.46 105.85) (end 178.3 105.85) (width 0.24) (layer F.Cu) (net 7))
 (segment (start 178.3 105.85) (end 178.6 106.15) (width 0.24) (layer F.Cu) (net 7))
 (segment (start 178.6 106.15) (end 178.6 107.65) (width 0.24) (layer F.Cu) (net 7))
 (segment (start 178.6 107.65) (end 178.3 107.95) (width 0.24) (layer F.Cu) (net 7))
 (segment (start 178.3 107.95) (end 175.6 107.95) (width 0.24) (layer F.Cu) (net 7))
 (segment (start 175.6 107.95) (end 175.1125 108.4375) (width 0.24) (layer F.Cu) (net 7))
 (segment (start 175.1125 108.4375) (end 175.1125 109.25) (width 0.24) (layer F.Cu) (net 7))
 (segment (start 170.65 109.8) (end 170 109.8) (width 0.24) (layer B.Cu) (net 6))
 (segment (start 158.3 107.7) (end 156.5 107.7) (width 0.24) (layer B.Cu) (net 6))
 (segment (start 170 109.8) (end 168.5 108.3) (width 0.24) (layer B.Cu) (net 6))
 (segment (start 168.5 108.3) (end 158.9 108.3) (width 0.24) (layer B.Cu) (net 6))
 (segment (start 158.9 108.3) (end 158.3 107.7) (width 0.24) (layer B.Cu) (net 6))
 (segment (start 170.65 109.8) (end 170.211594 109.8) (width 0.24) (layer F.Cu) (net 6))
 (segment (start 170.211594 109.8) (end 169.661594 109.25) (width 0.24) (layer F.Cu) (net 6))
 (segment (start 169.661594 109.25) (end 169.49 109.25) (width 0.24) (layer F.Cu) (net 6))
 (segment (start 169.49 109.25) (end 168.9 109.25) (width 0.24) (layer F.Cu) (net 6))
 (segment (start 171.5475 108.9525) (end 170.7 109.8) (width 0.24) (layer B.Cu) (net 6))
 (segment (start 170.7 109.8) (end 170.65 109.8) (width 0.24) (layer B.Cu) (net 6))
 (via (at 170.65 109.8) (size 0.62) (drill 0.31) (layers F.Cu B.Cu) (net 6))
 (segment (start 173.7 108.9525) (end 171.5475 108.9525) (width 0.24) (layer B.Cu) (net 6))
 (via (at 173.7 108.9525) (size 0.62) (drill 0.31) (layers F.Cu B.Cu) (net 6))
 (segment (start 173.7 107) (end 174.2 106.5) (width 0.24) (layer F.Cu) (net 6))
 (segment (start 174.2 106.5) (end 175.55 106.5) (width 0.24) (layer F.Cu) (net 6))
 (segment (start 173.7 108.9525) (end 173.7 107) (width 0.24) (layer F.Cu) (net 6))
 (segment (start 175.1125 109.75) (end 174.4975 109.75) (width 0.24) (layer F.Cu) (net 6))
 (segment (start 174.4975 109.75) (end 173.7 108.9525) (width 0.24) (layer F.Cu) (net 6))
 (segment (start 166.1 108.25) (end 166.1 102.65) (width 0.24) (layer F.Cu) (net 1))
 (segment (start 166.1 102.65) (end 166.1 101) (width 0.24) (layer F.Cu) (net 1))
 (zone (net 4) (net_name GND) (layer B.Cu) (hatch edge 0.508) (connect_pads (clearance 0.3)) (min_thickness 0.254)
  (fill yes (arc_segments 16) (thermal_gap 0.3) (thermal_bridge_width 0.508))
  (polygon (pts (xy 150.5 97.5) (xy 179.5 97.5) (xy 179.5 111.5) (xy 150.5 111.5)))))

